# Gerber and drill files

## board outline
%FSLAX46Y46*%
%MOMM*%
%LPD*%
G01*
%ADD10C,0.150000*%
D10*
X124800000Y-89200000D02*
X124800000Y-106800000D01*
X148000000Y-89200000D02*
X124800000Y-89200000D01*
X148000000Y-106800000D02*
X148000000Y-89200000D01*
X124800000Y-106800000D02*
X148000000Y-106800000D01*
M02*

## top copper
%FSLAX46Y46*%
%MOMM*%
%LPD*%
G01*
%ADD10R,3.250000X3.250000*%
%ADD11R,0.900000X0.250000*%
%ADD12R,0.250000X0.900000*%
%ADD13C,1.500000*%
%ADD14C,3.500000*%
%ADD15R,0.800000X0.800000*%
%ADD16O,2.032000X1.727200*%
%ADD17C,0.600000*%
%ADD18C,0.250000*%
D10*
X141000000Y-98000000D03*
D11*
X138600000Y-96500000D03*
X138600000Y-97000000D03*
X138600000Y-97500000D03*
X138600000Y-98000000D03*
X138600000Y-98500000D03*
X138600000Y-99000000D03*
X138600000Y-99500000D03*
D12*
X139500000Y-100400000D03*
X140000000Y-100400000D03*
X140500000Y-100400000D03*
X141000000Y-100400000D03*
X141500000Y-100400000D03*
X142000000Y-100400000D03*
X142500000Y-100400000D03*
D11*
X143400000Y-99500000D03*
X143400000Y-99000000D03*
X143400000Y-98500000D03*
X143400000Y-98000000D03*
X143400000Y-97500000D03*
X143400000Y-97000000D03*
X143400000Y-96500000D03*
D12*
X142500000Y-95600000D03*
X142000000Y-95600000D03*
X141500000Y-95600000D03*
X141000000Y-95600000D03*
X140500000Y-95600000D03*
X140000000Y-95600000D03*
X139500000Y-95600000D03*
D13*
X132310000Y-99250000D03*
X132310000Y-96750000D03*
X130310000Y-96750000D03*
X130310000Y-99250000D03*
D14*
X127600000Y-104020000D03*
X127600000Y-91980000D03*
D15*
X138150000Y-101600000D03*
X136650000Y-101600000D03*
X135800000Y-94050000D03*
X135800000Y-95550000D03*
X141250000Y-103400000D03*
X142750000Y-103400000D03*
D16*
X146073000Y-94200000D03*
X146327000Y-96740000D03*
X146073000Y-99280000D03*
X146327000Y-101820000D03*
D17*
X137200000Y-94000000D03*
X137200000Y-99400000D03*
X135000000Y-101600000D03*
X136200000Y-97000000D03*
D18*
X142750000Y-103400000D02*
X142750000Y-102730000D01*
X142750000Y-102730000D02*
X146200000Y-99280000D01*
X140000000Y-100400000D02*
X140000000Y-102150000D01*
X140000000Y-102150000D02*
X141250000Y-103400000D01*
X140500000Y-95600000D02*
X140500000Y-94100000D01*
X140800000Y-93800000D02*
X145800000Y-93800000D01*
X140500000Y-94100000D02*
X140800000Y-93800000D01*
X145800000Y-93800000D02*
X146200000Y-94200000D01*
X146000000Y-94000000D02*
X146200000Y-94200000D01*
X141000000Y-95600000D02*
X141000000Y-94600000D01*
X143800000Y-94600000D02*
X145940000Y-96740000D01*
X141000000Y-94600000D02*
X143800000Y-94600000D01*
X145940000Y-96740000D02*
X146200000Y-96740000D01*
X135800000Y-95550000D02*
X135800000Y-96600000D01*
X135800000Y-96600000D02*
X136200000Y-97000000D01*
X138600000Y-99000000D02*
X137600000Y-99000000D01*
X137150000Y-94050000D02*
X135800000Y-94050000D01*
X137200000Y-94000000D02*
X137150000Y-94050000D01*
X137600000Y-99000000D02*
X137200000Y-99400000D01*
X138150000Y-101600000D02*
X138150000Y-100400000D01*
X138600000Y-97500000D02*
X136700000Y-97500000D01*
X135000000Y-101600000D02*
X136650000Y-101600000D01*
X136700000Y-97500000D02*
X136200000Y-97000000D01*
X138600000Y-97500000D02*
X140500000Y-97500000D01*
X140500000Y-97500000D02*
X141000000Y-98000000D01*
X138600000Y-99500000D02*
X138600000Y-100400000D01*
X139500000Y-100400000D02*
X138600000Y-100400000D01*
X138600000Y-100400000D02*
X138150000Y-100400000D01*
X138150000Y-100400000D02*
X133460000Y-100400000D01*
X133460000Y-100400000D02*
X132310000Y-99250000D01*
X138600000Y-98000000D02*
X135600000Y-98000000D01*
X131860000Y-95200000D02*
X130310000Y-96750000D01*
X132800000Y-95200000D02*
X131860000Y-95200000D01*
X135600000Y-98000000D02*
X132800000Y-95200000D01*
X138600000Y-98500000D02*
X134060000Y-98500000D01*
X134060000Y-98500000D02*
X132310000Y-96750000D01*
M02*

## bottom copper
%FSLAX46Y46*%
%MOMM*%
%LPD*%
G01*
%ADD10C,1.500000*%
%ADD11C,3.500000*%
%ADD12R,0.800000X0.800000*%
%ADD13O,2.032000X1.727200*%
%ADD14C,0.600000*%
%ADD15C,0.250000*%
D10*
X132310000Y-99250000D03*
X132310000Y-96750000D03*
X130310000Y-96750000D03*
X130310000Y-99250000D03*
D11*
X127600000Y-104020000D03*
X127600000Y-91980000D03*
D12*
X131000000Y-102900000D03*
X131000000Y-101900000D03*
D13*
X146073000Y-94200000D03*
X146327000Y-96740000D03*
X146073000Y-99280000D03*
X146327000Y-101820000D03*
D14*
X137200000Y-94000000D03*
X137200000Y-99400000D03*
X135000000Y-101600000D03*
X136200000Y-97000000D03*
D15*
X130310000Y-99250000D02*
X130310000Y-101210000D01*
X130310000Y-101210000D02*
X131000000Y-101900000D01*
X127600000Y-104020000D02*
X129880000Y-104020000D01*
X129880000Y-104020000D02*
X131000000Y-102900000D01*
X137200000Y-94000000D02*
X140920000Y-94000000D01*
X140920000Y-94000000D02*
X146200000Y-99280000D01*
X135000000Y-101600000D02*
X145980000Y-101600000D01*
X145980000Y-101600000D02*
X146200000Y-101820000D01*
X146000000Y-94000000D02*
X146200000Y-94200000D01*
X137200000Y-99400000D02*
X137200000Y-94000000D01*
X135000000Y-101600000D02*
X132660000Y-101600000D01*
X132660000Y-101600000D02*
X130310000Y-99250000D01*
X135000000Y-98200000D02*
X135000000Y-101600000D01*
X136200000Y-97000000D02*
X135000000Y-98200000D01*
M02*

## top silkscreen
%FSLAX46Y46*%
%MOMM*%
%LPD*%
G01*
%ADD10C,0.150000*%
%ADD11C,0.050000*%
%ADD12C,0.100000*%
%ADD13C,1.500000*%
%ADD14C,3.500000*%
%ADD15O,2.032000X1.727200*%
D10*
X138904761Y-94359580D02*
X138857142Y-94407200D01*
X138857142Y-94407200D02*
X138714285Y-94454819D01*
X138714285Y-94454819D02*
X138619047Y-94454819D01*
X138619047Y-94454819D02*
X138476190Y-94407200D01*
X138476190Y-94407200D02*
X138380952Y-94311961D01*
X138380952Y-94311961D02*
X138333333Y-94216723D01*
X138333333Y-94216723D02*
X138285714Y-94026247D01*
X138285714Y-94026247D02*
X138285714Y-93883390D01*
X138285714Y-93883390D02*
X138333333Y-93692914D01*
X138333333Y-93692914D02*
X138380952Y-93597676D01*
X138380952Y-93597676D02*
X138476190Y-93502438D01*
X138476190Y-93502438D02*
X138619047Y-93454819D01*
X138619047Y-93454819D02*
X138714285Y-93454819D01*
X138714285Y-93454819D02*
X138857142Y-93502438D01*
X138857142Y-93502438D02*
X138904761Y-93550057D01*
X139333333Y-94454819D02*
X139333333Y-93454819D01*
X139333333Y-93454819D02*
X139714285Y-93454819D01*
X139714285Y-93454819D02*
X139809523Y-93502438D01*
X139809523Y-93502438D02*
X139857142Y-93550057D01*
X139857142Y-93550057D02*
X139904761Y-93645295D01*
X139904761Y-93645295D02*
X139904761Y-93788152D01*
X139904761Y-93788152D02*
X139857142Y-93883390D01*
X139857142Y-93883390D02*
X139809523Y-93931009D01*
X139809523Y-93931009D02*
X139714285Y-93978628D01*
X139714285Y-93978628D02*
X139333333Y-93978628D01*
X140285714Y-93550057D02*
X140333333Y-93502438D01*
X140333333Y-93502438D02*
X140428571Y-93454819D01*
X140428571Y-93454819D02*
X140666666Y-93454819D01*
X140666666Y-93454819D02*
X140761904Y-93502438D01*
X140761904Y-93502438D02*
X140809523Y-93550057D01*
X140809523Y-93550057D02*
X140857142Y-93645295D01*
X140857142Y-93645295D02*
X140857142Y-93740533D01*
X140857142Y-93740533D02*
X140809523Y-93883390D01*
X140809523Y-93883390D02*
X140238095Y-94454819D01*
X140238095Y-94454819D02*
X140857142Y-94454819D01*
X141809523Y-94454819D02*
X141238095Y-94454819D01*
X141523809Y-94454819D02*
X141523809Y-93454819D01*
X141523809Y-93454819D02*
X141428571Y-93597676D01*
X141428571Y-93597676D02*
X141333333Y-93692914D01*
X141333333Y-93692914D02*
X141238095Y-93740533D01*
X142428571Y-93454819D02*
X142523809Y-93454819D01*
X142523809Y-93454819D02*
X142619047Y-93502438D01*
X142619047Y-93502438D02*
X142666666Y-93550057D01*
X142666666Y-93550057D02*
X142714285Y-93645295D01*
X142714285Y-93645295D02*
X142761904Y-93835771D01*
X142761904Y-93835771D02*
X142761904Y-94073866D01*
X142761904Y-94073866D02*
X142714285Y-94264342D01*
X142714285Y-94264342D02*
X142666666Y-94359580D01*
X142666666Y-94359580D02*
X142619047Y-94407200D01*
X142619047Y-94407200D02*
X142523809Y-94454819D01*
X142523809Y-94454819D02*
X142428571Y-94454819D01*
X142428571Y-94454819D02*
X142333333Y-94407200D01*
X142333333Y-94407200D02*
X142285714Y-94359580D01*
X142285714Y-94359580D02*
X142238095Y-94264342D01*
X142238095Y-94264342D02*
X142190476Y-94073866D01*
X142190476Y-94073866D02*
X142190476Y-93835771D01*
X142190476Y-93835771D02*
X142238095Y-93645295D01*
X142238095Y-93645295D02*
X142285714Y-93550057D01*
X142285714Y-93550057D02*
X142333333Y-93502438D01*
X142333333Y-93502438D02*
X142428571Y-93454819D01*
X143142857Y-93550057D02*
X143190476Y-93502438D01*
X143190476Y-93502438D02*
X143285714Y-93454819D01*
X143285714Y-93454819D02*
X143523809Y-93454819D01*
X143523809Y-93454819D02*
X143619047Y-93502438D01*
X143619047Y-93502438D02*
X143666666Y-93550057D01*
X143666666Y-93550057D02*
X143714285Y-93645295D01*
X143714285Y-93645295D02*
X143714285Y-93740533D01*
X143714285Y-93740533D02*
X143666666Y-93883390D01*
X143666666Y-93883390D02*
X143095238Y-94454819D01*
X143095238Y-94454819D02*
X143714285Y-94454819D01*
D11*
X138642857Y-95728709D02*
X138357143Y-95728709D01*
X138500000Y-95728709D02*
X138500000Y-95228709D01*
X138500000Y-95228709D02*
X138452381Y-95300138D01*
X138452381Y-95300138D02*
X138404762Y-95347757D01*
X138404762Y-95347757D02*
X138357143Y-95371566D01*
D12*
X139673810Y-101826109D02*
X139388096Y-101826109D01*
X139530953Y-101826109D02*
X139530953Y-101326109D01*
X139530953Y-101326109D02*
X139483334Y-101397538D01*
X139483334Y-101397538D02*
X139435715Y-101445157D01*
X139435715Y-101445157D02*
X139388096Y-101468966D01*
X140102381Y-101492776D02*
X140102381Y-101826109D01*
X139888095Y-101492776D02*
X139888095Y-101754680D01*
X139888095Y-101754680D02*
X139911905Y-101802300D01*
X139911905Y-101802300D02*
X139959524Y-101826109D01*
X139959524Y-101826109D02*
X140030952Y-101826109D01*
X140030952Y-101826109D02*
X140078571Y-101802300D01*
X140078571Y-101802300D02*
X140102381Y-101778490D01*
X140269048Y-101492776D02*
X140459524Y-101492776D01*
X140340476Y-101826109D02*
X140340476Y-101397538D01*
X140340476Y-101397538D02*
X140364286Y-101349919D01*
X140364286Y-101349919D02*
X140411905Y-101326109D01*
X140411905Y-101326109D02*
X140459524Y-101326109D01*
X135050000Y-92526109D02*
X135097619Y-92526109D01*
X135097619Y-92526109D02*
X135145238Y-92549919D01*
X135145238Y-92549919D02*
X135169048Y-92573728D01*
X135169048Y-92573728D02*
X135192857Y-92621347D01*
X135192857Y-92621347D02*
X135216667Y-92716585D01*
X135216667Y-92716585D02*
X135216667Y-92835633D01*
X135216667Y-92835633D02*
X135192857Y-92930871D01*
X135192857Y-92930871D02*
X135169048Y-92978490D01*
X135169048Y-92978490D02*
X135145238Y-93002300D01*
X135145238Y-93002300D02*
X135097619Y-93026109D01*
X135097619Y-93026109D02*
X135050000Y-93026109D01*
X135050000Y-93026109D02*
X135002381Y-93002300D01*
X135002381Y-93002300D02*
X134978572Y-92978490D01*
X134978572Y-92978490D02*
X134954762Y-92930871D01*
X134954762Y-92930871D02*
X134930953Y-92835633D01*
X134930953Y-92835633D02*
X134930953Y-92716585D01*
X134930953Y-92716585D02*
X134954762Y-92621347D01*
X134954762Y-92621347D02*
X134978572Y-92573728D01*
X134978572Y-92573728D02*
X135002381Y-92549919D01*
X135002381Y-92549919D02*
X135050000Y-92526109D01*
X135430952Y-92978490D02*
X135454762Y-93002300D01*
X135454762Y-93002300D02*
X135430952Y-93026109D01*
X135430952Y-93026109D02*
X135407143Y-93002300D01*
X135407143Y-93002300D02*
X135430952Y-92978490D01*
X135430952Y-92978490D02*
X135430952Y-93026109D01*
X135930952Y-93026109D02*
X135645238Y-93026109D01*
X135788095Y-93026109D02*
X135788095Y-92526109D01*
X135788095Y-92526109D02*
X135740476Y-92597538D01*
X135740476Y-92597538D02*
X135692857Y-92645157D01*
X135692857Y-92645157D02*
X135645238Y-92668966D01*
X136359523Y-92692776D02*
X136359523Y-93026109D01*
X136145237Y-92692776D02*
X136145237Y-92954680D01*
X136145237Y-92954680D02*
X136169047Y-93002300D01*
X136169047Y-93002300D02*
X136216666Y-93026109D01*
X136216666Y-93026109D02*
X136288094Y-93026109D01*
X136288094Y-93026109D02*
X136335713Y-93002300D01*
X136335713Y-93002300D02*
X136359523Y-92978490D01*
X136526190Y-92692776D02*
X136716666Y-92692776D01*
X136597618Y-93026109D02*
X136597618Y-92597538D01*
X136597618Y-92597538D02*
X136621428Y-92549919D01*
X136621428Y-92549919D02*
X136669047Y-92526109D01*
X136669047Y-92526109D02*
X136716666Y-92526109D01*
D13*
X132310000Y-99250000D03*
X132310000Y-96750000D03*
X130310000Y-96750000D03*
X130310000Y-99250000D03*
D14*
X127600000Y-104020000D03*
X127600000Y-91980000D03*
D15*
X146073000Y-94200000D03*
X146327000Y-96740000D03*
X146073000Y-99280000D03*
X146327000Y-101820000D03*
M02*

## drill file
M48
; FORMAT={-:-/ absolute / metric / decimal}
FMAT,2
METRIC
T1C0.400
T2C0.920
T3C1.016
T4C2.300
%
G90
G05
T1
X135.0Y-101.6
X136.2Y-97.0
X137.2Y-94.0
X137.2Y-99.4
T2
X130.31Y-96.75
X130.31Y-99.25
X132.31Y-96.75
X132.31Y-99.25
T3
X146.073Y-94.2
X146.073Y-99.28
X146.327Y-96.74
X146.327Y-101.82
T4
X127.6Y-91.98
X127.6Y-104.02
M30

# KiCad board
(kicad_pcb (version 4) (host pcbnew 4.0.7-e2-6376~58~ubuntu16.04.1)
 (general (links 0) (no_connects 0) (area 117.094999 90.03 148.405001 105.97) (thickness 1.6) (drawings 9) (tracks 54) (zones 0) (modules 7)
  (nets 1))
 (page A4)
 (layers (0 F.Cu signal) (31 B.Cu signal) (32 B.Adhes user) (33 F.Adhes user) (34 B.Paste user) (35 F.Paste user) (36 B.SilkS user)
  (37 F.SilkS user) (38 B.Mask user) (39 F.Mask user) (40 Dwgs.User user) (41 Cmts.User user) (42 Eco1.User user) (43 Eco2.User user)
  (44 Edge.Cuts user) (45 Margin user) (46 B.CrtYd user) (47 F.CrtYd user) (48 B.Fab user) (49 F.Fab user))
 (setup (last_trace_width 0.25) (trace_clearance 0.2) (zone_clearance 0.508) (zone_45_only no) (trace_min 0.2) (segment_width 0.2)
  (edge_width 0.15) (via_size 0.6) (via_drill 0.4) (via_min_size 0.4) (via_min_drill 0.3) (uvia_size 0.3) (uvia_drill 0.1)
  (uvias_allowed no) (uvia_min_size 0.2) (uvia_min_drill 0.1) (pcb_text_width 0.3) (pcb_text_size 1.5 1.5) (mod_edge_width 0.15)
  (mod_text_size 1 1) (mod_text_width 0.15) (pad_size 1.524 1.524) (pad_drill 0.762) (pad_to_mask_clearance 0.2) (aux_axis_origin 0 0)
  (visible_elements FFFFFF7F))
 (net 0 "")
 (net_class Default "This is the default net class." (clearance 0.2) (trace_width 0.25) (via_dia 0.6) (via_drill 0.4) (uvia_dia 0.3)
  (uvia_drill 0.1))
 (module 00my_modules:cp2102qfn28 (layer F.Cu) (at 141 98)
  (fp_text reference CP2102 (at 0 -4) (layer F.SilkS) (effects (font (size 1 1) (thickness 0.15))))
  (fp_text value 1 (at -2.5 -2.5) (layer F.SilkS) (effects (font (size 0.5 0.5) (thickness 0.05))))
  (pad GND smd rect (at 0 0) (size 3.25 3.25) (layers F.Cu F.Paste F.Mask))
  (pad 1 smd rect (at -2.4 -1.5) (size 0.9 0.25) (layers F.Cu F.Paste F.Mask))
  (pad 2 smd rect (at -2.4 -1) (size 0.9 0.25) (layers F.Cu F.Paste F.Mask))
  (pad 3 smd rect (at -2.4 -0.5) (size 0.9 0.25) (layers F.Cu F.Paste F.Mask))
  (pad 4 smd rect (at -2.4 0) (size 0.9 0.25) (layers F.Cu F.Paste F.Mask))
  (pad 5 smd rect (at -2.4 0.5) (size 0.9 0.25) (layers F.Cu F.Paste F.Mask))
  (pad 6 smd rect (at -2.4 1) (size 0.9 0.25) (layers F.Cu F.Paste F.Mask))
  (pad 7 smd rect (at -2.4 1.5) (size 0.9 0.25) (layers F.Cu F.Paste F.Mask))
  (pad 8 smd rect (at -1.5 2.4) (size 0.25 0.9) (layers F.Cu F.Paste F.Mask))
  (pad 9 smd rect (at -1 2.4) (size 0.25 0.9) (layers F.Cu F.Paste F.Mask))
  (pad 10 smd rect (at -0.5 2.4) (size 0.25 0.9) (layers F.Cu F.Paste F.Mask))
  (pad 11 smd rect (at 0 2.4) (size 0.25 0.9) (layers F.Cu F.Paste F.Mask))
  (pad 12 smd rect (at 0.5 2.4) (size 0.25 0.9) (layers F.Cu F.Paste F.Mask))
  (pad 13 smd rect (at 1 2.4) (size 0.25 0.9) (layers F.Cu F.Paste F.Mask))
  (pad 14 smd rect (at 1.5 2.4) (size 0.25 0.9) (layers F.Cu F.Paste F.Mask))
  (pad 15 smd rect (at 2.4 1.5) (size 0.9 0.25) (layers F.Cu F.Paste F.Mask))
  (pad 16 smd rect (at 2.4 1) (size 0.9 0.25) (layers F.Cu F.Paste F.Mask))
  (pad 17 smd rect (at 2.4 0.5) (size 0.9 0.25) (layers F.Cu F.Paste F.Mask))
  (pad 18 smd rect (at 2.4 0) (size 0.9 0.25) (layers F.Cu F.Paste F.Mask))
  (pad 19 smd rect (at 2.4 -0.5) (size 0.9 0.25) (layers F.Cu F.Paste F.Mask))
  (pad 20 smd rect (at 2.4 -1) (size 0.9 0.25) (layers F.Cu F.Paste F.Mask))
  (pad 21 smd rect (at 2.4 -1.5) (size 0.9 0.25) (layers F.Cu F.Paste F.Mask))
  (pad 22 smd rect (at 1.5 -2.4) (size 0.25 0.9) (layers F.Cu F.Paste F.Mask))
  (pad 23 smd rect (at 1 -2.4) (size 0.25 0.9) (layers F.Cu F.Paste F.Mask))
  (pad 24 smd rect (at 0.5 -2.4) (size 0.25 0.9) (layers F.Cu F.Paste F.Mask))
  (pad 25 smd rect (at 0 -2.4) (size 0.25 0.9) (layers F.Cu F.Paste F.Mask))
  (pad 26 smd rect (at -0.5 -2.4) (size 0.25 0.9) (layers F.Cu F.Paste F.Mask))
  (pad 27 smd rect (at -1 -2.4) (size 0.25 0.9) (layers F.Cu F.Paste F.Mask))
  (pad 28 smd rect (at -1.5 -2.4) (size 0.25 0.9) (layers F.Cu F.Paste F.Mask)))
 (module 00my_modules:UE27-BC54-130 (layer F.Cu) (at 127.6 98 270)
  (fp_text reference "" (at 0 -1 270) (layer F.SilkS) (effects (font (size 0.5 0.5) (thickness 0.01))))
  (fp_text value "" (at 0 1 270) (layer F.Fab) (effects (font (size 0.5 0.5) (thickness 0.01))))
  (pad V thru_hole circle (at 1.25 -4.71 270) (size 1.5 1.5) (drill 0.92) (layers *.Cu *.Mask F.SilkS))
  (pad - thru_hole circle (at -1.25 -4.71 270) (size 1.5 1.5) (drill 0.92) (layers *.Cu *.Mask F.SilkS))
  (pad + thru_hole circle (at -1.25 -2.71 270) (size 1.5 1.5) (drill 0.92) (layers *.Cu *.Mask F.SilkS))
  (pad G thru_hole circle (at 1.25 -2.71 270) (size 1.5 1.5) (drill 0.92) (layers *.Cu *.Mask F.SilkS))
  (pad X thru_hole circle (at 6.02 0 270) (size 3.5 3.5) (drill 2.3) (layers *.Cu *.Mask F.SilkS))
  (pad X thru_hole circle (at -6.02 0 270) (size 3.5 3.5) (drill 2.3) (layers *.Cu *.Mask F.SilkS)))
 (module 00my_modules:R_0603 (layer F.Cu) (at 137.4 101.6 180)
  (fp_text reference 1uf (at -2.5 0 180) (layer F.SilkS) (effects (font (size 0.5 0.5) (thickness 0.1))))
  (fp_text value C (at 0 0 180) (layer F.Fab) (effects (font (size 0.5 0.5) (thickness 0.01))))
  (pad 1 smd rect (at -0.75 0 180) (size 0.8 0.8) (layers F.Cu F.Paste F.Mask))
  (pad 2 smd rect (at 0.75 0 180) (size 0.8 0.8) (layers F.Cu F.Paste F.Mask)))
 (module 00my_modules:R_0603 (layer F.Cu) (at 135.8 94.8 270)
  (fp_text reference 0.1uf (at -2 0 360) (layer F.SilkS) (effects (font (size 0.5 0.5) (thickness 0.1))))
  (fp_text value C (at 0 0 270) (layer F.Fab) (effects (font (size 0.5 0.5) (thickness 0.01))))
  (pad 1 smd rect (at -0.75 0 270) (size 0.8 0.8) (layers F.Cu F.Paste F.Mask))
  (pad 2 smd rect (at 0.75 0 270) (size 0.8 0.8) (layers F.Cu F.Paste F.Mask)))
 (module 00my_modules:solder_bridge (layer B.Cu) (at 131 102.4 90)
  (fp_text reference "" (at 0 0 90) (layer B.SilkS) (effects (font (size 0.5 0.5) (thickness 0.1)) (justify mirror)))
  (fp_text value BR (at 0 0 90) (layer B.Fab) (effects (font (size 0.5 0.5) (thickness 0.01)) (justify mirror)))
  (pad 1 smd rect (at -0.5 0 90) (size 0.8 0.8) (layers B.Cu B.Paste B.Mask))
  (pad 2 smd rect (at 0.5 0 90) (size 0.8 0.8) (layers B.Cu B.Paste B.Mask)))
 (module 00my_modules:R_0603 (layer F.Cu) (at 142 103.4)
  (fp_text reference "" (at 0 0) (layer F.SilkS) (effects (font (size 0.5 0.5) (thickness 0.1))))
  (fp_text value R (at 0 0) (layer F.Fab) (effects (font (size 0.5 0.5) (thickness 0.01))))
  (pad 1 smd rect (at -0.75 0) (size 0.8 0.8) (layers F.Cu F.Paste F.Mask))
  (pad 2 smd rect (at 0.75 0) (size 0.8 0.8) (layers F.Cu F.Paste F.Mask)))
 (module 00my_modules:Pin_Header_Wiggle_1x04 (layer F.Cu) (at 146.2 94.2)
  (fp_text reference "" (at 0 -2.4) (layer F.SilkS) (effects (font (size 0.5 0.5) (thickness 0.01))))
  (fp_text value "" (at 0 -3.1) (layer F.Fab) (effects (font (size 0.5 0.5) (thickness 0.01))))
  (pad 1 thru_hole oval (at -0.127 0) (size 2.032 1.7272) (drill 1.016) (layers *.Cu *.Mask F.SilkS))
  (pad 2 thru_hole oval (at 0.127 2.54) (size 2.032 1.7272) (drill 1.016) (layers *.Cu *.Mask F.SilkS))
  (pad 3 thru_hole oval (at -0.127 5.08) (size 2.032 1.7272) (drill 1.016) (layers *.Cu *.Mask F.SilkS))
  (pad 4 thru_hole oval (at 0.127 7.62) (size 2.032 1.7272) (drill 1.016) (layers *.Cu *.Mask F.SilkS)))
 (gr_line (start 124.8 89.2) (end 124.8 106.8) (angle 90) (layer Edge.Cuts) (width 0.15))
 (gr_line (start 148 89.2) (end 124.8 89.2) (angle 90) (layer Edge.Cuts) (width 0.15))
 (gr_line (start 148 106.8) (end 148 89.2) (angle 90) (layer Edge.Cuts) (width 0.15))
 (gr_line (start 124.8 106.8) (end 148 106.8) (angle 90) (layer Edge.Cuts) (width 0.15))
 (segment (start 142.75 103.4) (end 142.75 102.73) (width 0.25) (layer F.Cu) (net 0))
 (segment (start 142.75 102.73) (end 146.2 99.28) (width 0.25) (layer F.Cu) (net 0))
 (segment (start 140 100.4) (end 140 102.15) (width 0.25) (layer F.Cu) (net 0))
 (segment (start 140 102.15) (end 141.25 103.4) (width 0.25) (layer F.Cu) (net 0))
 (segment (start 140.5 95.6) (end 140.5 94.1) (width 0.25) (layer F.Cu) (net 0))
 (segment (start 140.8 93.8) (end 145.8 93.8) (width 0.25) (layer F.Cu) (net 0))
 (segment (start 140.5 94.1) (end 140.8 93.8) (width 0.25) (layer F.Cu) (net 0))
 (segment (start 145.8 93.8) (end 146.2 94.2) (width 0.25) (layer F.Cu) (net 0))
 (segment (start 130.31 99.25) (end 130.31 101.21) (width 0.25) (layer B.Cu) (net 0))
 (segment (start 130.31 101.21) (end 131 101.9) (width 0.25) (layer B.Cu) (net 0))
 (segment (start 127.6 104.02) (end 129.88 104.02) (width 0.25) (layer B.Cu) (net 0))
 (segment (start 129.88 104.02) (end 131 102.9) (width 0.25) (layer B.Cu) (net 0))
 (segment (start 137.2 94) (end 140.92 94) (width 0.25) (layer B.Cu) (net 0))
 (segment (start 140.92 94) (end 146.2 99.28) (width 0.25) (layer B.Cu) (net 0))
 (segment (start 146 94) (end 146.2 94.2) (width 0.25) (layer F.Cu) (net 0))
 (segment (start 141 95.6) (end 141 94.6) (width 0.25) (layer F.Cu) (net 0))
 (segment (start 143.8 94.6) (end 145.94 96.74) (width 0.25) (layer F.Cu) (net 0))
 (segment (start 141 94.6) (end 143.8 94.6) (width 0.25) (layer F.Cu) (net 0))
 (segment (start 145.94 96.74) (end 146.2 96.74) (width 0.25) (layer F.Cu) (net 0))
 (segment (start 135 101.6) (end 145.98 101.6) (width 0.25) (layer B.Cu) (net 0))
 (segment (start 145.98 101.6) (end 146.2 101.82) (width 0.25) (layer B.Cu) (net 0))
 (segment (start 146 94) (end 146.2 94.2) (width 0.25) (layer B.Cu) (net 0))
 (segment (start 135.8 95.55) (end 135.8 96.6) (width 0.25) (layer F.Cu) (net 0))
 (segment (start 135.8 96.6) (end 136.2 97) (width 0.25) (layer F.Cu) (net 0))
 (segment (start 138.6 99) (end 137.6 99) (width 0.25) (layer F.Cu) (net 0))
 (segment (start 137.15 94.05) (end 135.8 94.05) (width 0.25) (layer F.Cu) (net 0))
 (segment (start 137.2 94) (end 137.15 94.05) (width 0.25) (layer F.Cu) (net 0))
 (via (at 137.2 94) (size 0.6) (drill 0.4) (layers F.Cu B.Cu) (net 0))
 (segment (start 137.2 99.4) (end 137.2 94) (width 0.25) (layer B.Cu) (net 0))
 (via (at 137.2 99.4) (size 0.6) (drill 0.4) (layers F.Cu B.Cu) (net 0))
 (segment (start 137.6 99) (end 137.2 99.4) (width 0.25) (layer F.Cu) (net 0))
 (segment (start 135 101.6) (end 132.66 101.6) (width 0.25) (layer B.Cu) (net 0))
 (segment (start 132.66 101.6) (end 130.31 99.25) (width 0.25) (layer B.Cu) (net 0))
 (segment (start 138.15 101.6) (end 138.15 100.4) (width 0.25) (layer F.Cu) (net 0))
 (segment (start 138.6 97.5) (end 136.7 97.5) (width 0.25) (layer F.Cu) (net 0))
 (segment (start 135 101.6) (end 136.65 101.6) (width 0.25) (layer F.Cu) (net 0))
 (via (at 135 101.6) (size 0.6) (drill 0.4) (layers F.Cu B.Cu) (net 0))
 (segment (start 135 98.2) (end 135 101.6) (width 0.25) (layer B.Cu) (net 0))
 (segment (start 136.2 97) (end 135 98.2) (width 0.25) (layer B.Cu) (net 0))
 (via (at 136.2 97) (size 0.6) (drill 0.4) (layers F.Cu B.Cu) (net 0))
 (segment (start 136.7 97.5) (end 136.2 97) (width 0.25) (layer F.Cu) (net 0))
 (segment (start 138.6 97.5) (end 140.5 97.5) (width 0.25) (layer F.Cu) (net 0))
 (segment (start 140.5 97.5) (end 141 98) (width 0.25) (layer F.Cu) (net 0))
 (segment (start 138.6 99.5) (end 138.6 100.4) (width 0.25) (layer F.Cu) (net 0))
 (segment (start 139.5 100.4) (end 138.6 100.4) (width 0.25) (layer F.Cu) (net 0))
 (segment (start 138.6 100.4) (end 138.15 100.4) (width 0.25) (layer F.Cu) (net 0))
 (segment (start 138.15 100.4) (end 133.46 100.4) (width 0.25) (layer F.Cu) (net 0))
 (segment (start 133.46 100.4) (end 132.31 99.25) (width 0.25) (layer F.Cu) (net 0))
 (segment (start 138.6 98) (end 135.6 98) (width 0.25) (layer F.Cu) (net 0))
 (segment (start 131.86 95.2) (end 130.31 96.75) (width 0.25) (layer F.Cu) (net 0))
 (segment (start 132.8 95.2) (end 131.86 95.2) (width 0.25) (layer F.Cu) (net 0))
 (segment (start 135.6 98) (end 132.8 95.2) (width 0.25) (layer F.Cu) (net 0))
 (segment (start 138.6 98.5) (end 134.06 98.5) (width 0.25) (layer F.Cu) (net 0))
 (segment (start 134.06 98.5) (end 132.31 96.75) (width 0.25) (layer F.Cu) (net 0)))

